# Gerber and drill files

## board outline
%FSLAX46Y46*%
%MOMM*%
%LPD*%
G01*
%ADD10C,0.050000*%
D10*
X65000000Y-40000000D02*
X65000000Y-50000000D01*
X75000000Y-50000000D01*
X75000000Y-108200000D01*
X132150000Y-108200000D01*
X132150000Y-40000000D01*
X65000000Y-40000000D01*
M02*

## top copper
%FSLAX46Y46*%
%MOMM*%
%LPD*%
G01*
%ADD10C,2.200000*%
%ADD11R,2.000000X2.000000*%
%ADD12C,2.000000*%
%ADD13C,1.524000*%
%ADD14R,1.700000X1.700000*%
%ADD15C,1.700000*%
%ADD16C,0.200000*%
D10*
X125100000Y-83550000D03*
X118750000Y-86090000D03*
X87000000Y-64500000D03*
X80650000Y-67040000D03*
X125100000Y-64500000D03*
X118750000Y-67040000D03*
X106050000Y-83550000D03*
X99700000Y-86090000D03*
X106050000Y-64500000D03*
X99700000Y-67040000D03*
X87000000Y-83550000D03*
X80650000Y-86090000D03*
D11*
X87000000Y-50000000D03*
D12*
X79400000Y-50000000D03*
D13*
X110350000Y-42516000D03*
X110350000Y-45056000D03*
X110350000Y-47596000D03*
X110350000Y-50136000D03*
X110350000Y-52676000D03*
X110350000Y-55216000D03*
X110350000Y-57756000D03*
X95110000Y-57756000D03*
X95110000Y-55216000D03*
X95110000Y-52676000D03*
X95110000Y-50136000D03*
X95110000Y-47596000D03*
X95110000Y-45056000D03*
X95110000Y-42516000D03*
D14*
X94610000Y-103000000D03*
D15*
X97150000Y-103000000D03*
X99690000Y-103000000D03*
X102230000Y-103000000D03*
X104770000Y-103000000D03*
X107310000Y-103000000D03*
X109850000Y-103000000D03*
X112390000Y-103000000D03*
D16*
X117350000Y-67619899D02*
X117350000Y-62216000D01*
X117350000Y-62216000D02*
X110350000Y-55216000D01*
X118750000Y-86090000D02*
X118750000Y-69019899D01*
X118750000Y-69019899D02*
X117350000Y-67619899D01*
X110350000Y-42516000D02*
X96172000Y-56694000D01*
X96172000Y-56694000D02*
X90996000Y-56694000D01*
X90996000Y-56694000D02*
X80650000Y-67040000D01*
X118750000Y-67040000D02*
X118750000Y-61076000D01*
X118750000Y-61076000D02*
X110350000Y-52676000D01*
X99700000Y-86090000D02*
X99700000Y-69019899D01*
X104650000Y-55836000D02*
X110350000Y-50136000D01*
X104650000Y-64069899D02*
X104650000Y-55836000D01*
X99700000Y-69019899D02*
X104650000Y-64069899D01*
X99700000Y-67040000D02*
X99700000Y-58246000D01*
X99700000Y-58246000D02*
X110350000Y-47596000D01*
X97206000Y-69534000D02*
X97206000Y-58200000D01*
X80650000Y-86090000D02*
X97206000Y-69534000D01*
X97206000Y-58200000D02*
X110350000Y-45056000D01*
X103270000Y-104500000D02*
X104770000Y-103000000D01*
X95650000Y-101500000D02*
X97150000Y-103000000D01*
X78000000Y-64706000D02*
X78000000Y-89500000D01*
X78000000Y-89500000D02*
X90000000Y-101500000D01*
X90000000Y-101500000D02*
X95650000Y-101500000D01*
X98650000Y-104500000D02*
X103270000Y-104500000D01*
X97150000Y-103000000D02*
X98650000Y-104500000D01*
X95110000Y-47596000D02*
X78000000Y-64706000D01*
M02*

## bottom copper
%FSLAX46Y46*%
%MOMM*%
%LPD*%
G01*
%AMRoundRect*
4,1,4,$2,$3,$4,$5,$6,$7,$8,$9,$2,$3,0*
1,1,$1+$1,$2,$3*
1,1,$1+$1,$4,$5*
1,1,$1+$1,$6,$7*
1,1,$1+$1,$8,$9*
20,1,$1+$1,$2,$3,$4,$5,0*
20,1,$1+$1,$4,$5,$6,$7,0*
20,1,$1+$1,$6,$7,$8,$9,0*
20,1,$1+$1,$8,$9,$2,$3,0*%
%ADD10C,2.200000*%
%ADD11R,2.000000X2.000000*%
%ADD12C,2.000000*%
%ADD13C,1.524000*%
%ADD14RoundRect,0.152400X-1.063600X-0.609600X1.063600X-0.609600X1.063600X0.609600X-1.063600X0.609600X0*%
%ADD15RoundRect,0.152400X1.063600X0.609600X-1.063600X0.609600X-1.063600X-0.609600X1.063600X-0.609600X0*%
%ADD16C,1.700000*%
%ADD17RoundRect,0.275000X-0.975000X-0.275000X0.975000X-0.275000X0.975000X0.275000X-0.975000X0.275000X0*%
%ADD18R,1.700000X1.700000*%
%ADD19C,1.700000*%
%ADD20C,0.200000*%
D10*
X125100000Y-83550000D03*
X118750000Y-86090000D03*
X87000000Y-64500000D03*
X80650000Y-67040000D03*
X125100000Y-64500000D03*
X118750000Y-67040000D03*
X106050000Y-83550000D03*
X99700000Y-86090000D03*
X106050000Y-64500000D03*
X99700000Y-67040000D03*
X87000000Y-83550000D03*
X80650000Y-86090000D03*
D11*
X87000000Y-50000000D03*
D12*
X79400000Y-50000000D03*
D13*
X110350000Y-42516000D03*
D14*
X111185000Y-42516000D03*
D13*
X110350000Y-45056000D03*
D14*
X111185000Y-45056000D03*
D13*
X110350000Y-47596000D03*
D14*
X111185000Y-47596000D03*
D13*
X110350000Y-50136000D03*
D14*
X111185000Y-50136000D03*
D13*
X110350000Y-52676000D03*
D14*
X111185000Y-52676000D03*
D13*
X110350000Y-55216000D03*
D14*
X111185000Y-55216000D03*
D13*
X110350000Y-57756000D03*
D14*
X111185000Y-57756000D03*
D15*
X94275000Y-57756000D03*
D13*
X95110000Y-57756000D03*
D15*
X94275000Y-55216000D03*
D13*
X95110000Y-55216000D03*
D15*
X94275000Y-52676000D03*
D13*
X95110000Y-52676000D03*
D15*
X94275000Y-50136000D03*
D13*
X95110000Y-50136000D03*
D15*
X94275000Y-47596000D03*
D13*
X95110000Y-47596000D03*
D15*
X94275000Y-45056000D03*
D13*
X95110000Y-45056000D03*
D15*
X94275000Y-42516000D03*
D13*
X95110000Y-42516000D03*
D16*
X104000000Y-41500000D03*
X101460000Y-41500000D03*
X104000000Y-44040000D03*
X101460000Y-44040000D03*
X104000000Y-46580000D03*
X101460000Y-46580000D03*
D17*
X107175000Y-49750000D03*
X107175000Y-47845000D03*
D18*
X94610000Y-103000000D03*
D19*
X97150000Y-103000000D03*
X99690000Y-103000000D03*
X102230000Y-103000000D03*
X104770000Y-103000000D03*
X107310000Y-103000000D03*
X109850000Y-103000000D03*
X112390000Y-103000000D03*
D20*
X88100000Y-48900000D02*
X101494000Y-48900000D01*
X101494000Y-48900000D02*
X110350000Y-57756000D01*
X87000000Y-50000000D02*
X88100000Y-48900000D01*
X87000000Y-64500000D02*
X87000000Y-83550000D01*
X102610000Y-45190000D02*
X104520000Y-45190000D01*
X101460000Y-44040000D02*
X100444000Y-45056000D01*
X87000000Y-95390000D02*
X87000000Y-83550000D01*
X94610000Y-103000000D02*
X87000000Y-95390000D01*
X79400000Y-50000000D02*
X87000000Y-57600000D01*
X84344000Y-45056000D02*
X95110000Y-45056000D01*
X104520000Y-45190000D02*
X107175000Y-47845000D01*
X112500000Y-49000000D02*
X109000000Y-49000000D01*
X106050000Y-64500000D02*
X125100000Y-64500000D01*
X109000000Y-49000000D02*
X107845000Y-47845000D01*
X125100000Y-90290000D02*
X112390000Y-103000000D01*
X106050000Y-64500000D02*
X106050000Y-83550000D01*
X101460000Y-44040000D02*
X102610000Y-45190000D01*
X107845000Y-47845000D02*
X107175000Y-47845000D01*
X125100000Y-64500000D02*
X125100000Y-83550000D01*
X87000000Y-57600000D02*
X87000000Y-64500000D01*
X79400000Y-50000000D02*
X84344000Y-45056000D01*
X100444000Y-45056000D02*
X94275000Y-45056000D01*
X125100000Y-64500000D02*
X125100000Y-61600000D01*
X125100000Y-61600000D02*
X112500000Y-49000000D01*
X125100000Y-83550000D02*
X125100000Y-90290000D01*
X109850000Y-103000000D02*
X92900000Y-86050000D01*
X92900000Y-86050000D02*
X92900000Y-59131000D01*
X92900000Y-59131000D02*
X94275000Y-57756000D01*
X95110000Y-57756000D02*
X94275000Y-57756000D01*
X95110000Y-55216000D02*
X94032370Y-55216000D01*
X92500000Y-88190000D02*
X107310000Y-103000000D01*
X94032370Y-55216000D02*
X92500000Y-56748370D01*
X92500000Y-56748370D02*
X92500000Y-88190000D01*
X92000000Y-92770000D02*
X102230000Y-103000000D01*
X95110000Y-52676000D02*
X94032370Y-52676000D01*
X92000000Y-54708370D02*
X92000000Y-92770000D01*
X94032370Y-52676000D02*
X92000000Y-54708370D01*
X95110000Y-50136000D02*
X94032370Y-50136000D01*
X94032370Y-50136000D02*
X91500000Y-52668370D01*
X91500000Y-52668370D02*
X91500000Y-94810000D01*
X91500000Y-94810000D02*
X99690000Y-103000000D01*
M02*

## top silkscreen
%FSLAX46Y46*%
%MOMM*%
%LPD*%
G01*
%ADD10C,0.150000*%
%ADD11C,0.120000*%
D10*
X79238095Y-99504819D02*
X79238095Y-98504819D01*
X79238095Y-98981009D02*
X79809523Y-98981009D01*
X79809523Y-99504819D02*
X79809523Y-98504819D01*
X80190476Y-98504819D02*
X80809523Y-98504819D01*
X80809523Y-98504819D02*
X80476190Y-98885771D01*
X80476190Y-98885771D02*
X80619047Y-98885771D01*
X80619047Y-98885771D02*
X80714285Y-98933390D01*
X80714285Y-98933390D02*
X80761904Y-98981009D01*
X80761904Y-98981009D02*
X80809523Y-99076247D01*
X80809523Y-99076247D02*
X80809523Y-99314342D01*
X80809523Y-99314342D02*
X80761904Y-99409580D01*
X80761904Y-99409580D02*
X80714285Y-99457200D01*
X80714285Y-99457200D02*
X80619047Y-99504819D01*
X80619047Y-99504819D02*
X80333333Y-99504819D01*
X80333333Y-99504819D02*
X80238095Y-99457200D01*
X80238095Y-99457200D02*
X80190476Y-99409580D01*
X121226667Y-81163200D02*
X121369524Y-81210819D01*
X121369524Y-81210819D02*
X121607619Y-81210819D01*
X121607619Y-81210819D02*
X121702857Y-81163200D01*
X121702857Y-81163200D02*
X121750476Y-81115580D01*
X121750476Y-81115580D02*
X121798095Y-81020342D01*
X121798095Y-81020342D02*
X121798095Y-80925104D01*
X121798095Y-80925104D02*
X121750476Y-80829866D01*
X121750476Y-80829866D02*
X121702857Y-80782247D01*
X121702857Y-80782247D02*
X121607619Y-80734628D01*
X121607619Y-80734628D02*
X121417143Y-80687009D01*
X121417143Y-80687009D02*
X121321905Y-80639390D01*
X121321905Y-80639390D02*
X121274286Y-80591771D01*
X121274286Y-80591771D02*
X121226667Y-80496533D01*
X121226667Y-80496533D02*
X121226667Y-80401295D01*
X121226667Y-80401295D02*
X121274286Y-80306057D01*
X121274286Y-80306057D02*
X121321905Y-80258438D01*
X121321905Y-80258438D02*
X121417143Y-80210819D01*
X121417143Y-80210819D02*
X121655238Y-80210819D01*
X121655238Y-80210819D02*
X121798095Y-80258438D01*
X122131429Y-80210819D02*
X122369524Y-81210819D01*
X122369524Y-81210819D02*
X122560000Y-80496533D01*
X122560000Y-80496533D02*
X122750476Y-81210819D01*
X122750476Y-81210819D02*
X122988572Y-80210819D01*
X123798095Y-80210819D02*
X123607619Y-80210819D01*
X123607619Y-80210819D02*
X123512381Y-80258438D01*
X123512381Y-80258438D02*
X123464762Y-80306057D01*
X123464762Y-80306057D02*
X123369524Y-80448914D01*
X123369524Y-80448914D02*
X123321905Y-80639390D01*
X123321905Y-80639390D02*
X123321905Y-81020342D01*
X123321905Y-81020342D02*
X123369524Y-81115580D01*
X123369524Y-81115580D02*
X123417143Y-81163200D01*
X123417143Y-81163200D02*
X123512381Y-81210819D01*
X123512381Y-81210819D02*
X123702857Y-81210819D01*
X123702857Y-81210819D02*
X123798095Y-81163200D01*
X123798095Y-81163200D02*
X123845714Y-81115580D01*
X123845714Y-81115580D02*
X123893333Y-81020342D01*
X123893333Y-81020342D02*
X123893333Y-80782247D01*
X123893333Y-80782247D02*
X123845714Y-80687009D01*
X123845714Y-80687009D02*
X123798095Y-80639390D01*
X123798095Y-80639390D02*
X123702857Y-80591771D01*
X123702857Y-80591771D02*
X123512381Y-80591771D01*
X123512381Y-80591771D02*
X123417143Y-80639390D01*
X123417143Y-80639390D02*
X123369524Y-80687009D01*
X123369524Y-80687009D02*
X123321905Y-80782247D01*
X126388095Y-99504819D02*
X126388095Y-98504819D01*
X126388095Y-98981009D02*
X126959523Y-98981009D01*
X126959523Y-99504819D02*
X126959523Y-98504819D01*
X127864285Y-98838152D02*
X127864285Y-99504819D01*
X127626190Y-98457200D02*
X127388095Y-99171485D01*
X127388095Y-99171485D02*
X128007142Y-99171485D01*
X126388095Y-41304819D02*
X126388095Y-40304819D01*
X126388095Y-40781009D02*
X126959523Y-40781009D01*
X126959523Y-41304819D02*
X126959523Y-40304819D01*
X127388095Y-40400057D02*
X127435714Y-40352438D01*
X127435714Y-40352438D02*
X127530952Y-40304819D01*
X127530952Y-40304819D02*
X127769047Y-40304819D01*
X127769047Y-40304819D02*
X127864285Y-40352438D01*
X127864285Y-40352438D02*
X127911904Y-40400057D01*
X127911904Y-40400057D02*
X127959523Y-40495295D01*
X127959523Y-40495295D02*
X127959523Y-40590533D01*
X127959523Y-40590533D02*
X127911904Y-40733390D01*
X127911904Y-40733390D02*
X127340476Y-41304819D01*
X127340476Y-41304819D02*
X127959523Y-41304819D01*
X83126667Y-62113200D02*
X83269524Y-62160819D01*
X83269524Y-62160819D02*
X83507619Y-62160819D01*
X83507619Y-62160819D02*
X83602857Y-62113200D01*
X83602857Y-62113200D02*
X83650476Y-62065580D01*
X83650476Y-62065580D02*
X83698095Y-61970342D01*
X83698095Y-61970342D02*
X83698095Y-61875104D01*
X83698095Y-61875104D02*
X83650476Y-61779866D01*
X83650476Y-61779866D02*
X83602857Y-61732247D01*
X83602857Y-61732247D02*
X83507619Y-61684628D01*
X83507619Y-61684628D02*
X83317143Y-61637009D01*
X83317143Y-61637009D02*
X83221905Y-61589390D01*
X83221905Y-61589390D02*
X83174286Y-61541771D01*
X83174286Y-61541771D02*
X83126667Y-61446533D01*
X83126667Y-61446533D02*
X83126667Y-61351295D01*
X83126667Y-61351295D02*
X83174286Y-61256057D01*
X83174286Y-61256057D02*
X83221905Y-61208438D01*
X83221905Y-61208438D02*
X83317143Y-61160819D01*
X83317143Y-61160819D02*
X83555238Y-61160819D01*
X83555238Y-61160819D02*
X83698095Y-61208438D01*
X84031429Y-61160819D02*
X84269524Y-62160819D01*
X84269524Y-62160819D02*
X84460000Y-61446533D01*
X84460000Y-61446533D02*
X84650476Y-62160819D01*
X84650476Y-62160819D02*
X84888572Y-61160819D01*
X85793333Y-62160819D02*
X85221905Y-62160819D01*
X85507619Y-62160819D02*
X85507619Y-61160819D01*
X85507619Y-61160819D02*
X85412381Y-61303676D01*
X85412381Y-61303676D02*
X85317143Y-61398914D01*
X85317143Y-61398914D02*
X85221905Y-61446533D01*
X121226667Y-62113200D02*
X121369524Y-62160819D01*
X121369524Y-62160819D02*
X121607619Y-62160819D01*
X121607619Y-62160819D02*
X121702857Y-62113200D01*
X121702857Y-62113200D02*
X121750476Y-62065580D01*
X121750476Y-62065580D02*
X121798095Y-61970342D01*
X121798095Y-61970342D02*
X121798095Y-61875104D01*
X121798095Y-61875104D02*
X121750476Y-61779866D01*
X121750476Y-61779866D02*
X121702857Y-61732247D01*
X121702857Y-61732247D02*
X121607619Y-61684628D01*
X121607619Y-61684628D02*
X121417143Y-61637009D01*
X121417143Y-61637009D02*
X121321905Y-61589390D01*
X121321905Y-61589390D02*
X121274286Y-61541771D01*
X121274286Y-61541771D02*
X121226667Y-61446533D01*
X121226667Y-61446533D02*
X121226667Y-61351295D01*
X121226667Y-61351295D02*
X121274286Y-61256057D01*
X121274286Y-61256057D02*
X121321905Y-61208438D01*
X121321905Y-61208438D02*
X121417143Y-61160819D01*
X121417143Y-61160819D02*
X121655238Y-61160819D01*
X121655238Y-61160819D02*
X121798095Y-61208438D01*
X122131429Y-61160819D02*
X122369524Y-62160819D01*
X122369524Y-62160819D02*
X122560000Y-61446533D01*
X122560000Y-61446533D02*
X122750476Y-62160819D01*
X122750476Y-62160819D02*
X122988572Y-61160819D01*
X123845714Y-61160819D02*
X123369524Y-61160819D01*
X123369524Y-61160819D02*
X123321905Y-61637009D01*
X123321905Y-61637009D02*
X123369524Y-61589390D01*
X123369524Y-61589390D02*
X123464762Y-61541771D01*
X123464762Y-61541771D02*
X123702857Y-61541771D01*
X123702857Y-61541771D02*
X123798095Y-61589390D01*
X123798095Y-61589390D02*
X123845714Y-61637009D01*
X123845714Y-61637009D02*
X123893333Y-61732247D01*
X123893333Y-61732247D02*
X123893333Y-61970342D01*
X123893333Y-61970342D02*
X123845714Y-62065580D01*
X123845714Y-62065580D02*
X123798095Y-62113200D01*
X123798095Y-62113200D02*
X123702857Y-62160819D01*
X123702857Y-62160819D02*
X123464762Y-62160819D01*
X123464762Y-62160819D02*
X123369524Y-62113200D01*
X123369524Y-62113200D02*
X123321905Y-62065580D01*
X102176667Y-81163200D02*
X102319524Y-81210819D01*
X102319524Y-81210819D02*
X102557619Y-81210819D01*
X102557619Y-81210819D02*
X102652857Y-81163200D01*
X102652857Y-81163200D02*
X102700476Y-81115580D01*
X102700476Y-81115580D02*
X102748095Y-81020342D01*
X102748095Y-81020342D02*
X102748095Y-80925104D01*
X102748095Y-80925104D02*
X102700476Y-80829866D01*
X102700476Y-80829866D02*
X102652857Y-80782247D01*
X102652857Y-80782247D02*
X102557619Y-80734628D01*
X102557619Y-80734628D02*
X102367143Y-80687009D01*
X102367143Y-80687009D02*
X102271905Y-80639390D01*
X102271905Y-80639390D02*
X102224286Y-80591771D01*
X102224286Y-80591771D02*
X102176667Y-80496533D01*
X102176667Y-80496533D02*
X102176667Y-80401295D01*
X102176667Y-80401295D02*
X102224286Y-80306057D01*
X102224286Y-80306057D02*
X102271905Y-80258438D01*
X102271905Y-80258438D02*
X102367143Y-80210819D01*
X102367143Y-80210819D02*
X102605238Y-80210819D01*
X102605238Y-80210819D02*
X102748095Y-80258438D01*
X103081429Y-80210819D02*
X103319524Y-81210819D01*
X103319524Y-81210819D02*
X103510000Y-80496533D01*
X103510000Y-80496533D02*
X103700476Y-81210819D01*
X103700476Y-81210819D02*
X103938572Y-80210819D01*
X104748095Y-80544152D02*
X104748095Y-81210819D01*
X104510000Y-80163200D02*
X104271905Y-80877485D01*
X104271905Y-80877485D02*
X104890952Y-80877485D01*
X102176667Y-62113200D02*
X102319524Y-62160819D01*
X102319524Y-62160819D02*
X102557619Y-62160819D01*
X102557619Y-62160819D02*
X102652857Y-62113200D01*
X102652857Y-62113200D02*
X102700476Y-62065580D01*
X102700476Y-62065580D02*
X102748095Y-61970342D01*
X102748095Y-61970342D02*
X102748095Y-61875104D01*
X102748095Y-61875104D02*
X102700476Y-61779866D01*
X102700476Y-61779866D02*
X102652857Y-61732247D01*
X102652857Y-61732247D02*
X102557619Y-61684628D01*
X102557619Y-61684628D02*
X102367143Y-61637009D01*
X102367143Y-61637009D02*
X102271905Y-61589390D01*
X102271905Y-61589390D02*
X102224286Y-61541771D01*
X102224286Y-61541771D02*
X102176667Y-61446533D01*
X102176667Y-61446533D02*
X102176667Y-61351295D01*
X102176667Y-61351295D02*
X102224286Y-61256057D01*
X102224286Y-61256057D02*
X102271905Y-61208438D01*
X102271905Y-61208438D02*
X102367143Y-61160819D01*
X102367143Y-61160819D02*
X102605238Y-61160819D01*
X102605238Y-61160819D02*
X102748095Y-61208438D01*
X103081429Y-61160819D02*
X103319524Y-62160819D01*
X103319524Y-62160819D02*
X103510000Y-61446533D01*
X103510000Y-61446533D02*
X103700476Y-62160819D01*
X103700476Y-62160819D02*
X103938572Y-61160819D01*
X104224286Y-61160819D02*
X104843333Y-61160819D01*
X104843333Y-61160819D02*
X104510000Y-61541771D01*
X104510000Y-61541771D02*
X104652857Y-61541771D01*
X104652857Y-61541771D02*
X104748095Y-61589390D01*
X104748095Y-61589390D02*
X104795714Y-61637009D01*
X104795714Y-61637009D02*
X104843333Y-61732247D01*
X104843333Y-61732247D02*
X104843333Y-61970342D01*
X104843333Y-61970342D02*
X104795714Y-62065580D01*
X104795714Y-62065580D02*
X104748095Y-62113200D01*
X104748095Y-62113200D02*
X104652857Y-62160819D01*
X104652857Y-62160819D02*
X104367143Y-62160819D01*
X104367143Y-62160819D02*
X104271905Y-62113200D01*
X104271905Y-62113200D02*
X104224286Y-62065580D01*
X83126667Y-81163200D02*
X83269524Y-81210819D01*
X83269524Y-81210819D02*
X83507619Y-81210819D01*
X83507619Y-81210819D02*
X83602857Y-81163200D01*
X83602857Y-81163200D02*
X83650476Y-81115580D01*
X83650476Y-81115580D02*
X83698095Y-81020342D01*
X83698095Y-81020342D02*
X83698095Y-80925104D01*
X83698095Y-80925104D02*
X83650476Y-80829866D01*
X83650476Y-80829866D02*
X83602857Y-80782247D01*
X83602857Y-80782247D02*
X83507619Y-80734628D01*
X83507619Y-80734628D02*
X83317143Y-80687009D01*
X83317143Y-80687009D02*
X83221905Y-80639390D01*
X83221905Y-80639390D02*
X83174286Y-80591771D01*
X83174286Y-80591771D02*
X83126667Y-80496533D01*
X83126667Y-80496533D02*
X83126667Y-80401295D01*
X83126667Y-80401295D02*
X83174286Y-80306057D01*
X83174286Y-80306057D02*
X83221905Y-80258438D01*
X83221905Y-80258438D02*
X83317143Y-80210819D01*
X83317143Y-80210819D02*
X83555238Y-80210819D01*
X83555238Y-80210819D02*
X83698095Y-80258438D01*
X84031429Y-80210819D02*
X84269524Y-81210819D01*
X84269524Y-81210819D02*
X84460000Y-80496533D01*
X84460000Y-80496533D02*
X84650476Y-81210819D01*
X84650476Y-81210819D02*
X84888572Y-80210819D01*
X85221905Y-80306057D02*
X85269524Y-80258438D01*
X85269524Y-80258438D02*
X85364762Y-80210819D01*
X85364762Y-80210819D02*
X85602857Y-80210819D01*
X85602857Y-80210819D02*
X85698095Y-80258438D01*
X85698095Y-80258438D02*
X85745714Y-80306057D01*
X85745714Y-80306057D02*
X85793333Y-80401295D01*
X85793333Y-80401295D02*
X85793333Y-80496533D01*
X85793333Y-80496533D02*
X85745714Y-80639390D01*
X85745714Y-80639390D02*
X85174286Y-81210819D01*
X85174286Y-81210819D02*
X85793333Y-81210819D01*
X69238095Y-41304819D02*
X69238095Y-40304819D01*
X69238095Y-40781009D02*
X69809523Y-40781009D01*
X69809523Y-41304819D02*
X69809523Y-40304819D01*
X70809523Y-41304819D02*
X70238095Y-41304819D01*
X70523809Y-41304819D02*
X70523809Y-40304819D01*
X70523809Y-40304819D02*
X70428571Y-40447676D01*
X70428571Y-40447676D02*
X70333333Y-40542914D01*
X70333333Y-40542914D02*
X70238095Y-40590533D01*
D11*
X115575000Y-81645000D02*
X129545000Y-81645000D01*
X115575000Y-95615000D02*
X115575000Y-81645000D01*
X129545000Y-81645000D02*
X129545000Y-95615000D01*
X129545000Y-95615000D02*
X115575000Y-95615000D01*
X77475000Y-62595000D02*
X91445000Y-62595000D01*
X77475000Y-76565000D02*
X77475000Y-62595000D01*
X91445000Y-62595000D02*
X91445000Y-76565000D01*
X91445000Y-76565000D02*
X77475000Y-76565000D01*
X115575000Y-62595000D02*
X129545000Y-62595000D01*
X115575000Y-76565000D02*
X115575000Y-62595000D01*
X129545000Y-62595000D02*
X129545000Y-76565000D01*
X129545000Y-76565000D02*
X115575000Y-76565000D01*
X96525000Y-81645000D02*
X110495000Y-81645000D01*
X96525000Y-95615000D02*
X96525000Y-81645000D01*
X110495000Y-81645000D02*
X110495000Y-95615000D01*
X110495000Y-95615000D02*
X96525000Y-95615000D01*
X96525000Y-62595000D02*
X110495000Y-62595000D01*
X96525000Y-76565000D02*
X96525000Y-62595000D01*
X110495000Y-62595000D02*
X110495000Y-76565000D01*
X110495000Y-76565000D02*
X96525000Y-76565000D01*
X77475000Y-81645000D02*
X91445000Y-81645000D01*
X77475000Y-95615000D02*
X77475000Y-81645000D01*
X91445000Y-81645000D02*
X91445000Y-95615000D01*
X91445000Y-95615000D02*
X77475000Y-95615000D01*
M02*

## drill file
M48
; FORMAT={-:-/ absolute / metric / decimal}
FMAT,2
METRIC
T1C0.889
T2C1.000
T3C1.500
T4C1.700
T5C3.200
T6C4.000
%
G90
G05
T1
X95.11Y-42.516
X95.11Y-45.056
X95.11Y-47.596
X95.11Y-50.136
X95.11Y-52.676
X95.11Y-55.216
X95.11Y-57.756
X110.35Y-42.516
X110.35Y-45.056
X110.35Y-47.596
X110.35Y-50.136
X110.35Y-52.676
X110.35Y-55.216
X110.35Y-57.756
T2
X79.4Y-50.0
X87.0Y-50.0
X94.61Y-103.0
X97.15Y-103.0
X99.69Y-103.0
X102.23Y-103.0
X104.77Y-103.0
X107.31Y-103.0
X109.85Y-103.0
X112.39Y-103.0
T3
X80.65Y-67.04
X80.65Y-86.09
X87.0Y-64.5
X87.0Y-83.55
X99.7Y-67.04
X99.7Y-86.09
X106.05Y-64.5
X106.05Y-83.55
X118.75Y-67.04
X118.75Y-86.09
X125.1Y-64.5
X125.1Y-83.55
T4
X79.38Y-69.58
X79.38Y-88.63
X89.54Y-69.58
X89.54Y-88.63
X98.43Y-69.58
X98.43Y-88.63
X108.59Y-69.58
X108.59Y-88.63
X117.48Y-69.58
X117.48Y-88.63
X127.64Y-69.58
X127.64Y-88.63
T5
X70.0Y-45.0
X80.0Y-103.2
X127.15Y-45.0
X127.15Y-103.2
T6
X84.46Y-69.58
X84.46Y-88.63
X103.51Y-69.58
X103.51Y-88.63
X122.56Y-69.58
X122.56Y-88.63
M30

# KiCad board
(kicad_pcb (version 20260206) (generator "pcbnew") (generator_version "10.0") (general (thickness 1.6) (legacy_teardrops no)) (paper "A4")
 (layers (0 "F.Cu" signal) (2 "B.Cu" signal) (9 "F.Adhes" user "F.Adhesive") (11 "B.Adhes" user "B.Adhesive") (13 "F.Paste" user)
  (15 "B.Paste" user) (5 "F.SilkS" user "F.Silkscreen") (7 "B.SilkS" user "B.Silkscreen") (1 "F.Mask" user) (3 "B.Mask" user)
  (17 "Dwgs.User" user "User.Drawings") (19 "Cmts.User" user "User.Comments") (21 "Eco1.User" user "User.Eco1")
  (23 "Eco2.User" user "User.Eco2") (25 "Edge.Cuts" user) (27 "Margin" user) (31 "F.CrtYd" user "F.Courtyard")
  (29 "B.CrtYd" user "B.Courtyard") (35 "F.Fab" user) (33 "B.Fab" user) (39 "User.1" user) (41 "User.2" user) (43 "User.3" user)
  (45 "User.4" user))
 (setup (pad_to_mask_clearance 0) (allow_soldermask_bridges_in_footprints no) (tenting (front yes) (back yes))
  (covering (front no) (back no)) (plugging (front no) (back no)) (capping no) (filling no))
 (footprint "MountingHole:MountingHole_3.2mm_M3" (layer "F.Cu") (at 80 103.2)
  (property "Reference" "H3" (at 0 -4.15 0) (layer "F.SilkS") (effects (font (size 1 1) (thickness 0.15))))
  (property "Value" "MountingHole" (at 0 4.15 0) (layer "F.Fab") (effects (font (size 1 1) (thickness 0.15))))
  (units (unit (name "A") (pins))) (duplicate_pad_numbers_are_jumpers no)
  (pad "" np_thru_hole circle (at 0 0) (size 3.2 3.2) (drill 3.2) (layers "*.Cu" "*.Mask")))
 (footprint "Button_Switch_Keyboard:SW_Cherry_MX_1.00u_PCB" (layer "F.Cu") (at 125.1 83.55)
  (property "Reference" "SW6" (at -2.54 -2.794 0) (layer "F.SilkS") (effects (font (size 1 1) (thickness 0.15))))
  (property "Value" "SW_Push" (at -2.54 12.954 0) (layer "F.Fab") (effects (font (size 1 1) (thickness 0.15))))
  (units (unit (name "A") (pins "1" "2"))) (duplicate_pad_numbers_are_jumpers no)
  (fp_line (start -9.525 -1.905) (end 4.445 -1.905) (stroke (width 0.12) (type solid)) (layer "F.SilkS"))
  (fp_line (start -9.525 12.065) (end -9.525 -1.905) (stroke (width 0.12) (type solid)) (layer "F.SilkS"))
  (fp_line (start 4.445 -1.905) (end 4.445 12.065) (stroke (width 0.12) (type solid)) (layer "F.SilkS"))
  (fp_line (start 4.445 12.065) (end -9.525 12.065) (stroke (width 0.12) (type solid)) (layer "F.SilkS"))
  (pad "" np_thru_hole circle (at -7.62 5.08) (size 1.7 1.7) (drill 1.7) (layers "*.Cu" "*.Mask"))
  (pad "" np_thru_hole circle (at -2.54 5.08) (size 4 4) (drill 4) (layers "*.Cu" "*.Mask"))
  (pad "" np_thru_hole circle (at 2.54 5.08) (size 1.7 1.7) (drill 1.7) (layers "*.Cu" "*.Mask"))
  (pad "1" thru_hole circle (at 0 0) (size 2.2 2.2) (drill 1.5) (layers "*.Cu" "*.Mask") (remove_unused_layers no) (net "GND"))
  (pad "2" thru_hole circle (at -6.35 2.54) (size 2.2 2.2) (drill 1.5) (layers "*.Cu" "*.Mask") (remove_unused_layers no)
   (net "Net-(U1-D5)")))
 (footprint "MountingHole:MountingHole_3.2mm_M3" (layer "F.Cu") (at 127.15 103.2)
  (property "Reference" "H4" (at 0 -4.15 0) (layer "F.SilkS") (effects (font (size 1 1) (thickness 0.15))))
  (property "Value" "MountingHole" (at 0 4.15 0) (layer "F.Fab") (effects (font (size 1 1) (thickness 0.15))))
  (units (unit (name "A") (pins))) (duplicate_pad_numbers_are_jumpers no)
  (pad "" np_thru_hole circle (at 0 0) (size 3.2 3.2) (drill 3.2) (layers "*.Cu" "*.Mask")))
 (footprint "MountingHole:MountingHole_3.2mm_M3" (layer "F.Cu") (at 127.15 45)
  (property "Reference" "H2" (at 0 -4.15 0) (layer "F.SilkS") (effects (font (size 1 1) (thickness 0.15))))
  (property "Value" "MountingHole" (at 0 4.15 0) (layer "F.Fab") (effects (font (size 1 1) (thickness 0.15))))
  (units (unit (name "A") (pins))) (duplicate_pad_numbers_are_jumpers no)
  (pad "" np_thru_hole circle (at 0 0) (size 3.2 3.2) (drill 3.2) (layers "*.Cu" "*.Mask")))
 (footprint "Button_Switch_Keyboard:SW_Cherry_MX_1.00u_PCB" (layer "F.Cu") (at 87 64.5)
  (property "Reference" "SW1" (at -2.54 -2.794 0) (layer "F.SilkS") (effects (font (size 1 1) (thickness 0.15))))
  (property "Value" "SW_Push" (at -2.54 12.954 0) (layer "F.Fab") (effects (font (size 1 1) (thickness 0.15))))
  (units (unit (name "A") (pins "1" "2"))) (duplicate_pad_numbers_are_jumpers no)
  (fp_line (start -9.525 -1.905) (end 4.445 -1.905) (stroke (width 0.12) (type solid)) (layer "F.SilkS"))
  (fp_line (start -9.525 12.065) (end -9.525 -1.905) (stroke (width 0.12) (type solid)) (layer "F.SilkS"))
  (fp_line (start 4.445 -1.905) (end 4.445 12.065) (stroke (width 0.12) (type solid)) (layer "F.SilkS"))
  (fp_line (start 4.445 12.065) (end -9.525 12.065) (stroke (width 0.12) (type solid)) (layer "F.SilkS"))
  (pad "" np_thru_hole circle (at -7.62 5.08) (size 1.7 1.7) (drill 1.7) (layers "*.Cu" "*.Mask"))
  (pad "" np_thru_hole circle (at -2.54 5.08) (size 4 4) (drill 4) (layers "*.Cu" "*.Mask"))
  (pad "" np_thru_hole circle (at 2.54 5.08) (size 1.7 1.7) (drill 1.7) (layers "*.Cu" "*.Mask"))
  (pad "1" thru_hole circle (at 0 0) (size 2.2 2.2) (drill 1.5) (layers "*.Cu" "*.Mask") (remove_unused_layers no) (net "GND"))
  (pad "2" thru_hole circle (at -6.35 2.54) (size 2.2 2.2) (drill 1.5) (layers "*.Cu" "*.Mask") (remove_unused_layers no)
   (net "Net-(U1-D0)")))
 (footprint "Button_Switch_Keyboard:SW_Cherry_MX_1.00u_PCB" (layer "F.Cu") (at 125.1 64.5)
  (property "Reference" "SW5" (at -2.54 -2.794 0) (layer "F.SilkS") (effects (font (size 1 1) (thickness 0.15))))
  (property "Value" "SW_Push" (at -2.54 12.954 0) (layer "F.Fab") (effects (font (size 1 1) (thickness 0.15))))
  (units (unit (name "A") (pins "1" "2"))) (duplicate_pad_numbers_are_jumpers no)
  (fp_line (start -9.525 -1.905) (end 4.445 -1.905) (stroke (width 0.12) (type solid)) (layer "F.SilkS"))
  (fp_line (start -9.525 12.065) (end -9.525 -1.905) (stroke (width 0.12) (type solid)) (layer "F.SilkS"))
  (fp_line (start 4.445 -1.905) (end 4.445 12.065) (stroke (width 0.12) (type solid)) (layer "F.SilkS"))
  (fp_line (start 4.445 12.065) (end -9.525 12.065) (stroke (width 0.12) (type solid)) (layer "F.SilkS"))
  (pad "" np_thru_hole circle (at -7.62 5.08) (size 1.7 1.7) (drill 1.7) (layers "*.Cu" "*.Mask"))
  (pad "" np_thru_hole circle (at -2.54 5.08) (size 4 4) (drill 4) (layers "*.Cu" "*.Mask"))
  (pad "" np_thru_hole circle (at 2.54 5.08) (size 1.7 1.7) (drill 1.7) (layers "*.Cu" "*.Mask"))
  (pad "1" thru_hole circle (at 0 0) (size 2.2 2.2) (drill 1.5) (layers "*.Cu" "*.Mask") (remove_unused_layers no) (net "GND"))
  (pad "2" thru_hole circle (at -6.35 2.54) (size 2.2 2.2) (drill 1.5) (layers "*.Cu" "*.Mask") (remove_unused_layers no)
   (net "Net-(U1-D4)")))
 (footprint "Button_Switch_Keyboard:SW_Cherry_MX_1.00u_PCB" (layer "F.Cu") (at 106.05 83.55)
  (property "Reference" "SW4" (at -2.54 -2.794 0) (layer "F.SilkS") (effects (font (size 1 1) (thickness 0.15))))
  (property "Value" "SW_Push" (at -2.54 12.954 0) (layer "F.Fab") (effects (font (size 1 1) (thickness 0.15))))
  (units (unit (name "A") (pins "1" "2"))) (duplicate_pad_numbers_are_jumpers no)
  (fp_line (start -9.525 -1.905) (end 4.445 -1.905) (stroke (width 0.12) (type solid)) (layer "F.SilkS"))
  (fp_line (start -9.525 12.065) (end -9.525 -1.905) (stroke (width 0.12) (type solid)) (layer "F.SilkS"))
  (fp_line (start 4.445 -1.905) (end 4.445 12.065) (stroke (width 0.12) (type solid)) (layer "F.SilkS"))
  (fp_line (start 4.445 12.065) (end -9.525 12.065) (stroke (width 0.12) (type solid)) (layer "F.SilkS"))
  (pad "" np_thru_hole circle (at -7.62 5.08) (size 1.7 1.7) (drill 1.7) (layers "*.Cu" "*.Mask"))
  (pad "" np_thru_hole circle (at -2.54 5.08) (size 4 4) (drill 4) (layers "*.Cu" "*.Mask"))
  (pad "" np_thru_hole circle (at 2.54 5.08) (size 1.7 1.7) (drill 1.7) (layers "*.Cu" "*.Mask"))
  (pad "1" thru_hole circle (at 0 0) (size 2.2 2.2) (drill 1.5) (layers "*.Cu" "*.Mask") (remove_unused_layers no) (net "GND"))
  (pad "2" thru_hole circle (at -6.35 2.54) (size 2.2 2.2) (drill 1.5) (layers "*.Cu" "*.Mask") (remove_unused_layers no)
   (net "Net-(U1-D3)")))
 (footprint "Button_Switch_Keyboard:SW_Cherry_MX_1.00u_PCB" (layer "F.Cu") (at 106.05 64.5)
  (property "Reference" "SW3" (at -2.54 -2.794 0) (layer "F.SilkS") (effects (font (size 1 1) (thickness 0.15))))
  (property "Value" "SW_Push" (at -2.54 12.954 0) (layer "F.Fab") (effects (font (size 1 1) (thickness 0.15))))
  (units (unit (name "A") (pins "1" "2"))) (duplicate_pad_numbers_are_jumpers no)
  (fp_line (start -9.525 -1.905) (end 4.445 -1.905) (stroke (width 0.12) (type solid)) (layer "F.SilkS"))
  (fp_line (start -9.525 12.065) (end -9.525 -1.905) (stroke (width 0.12) (type solid)) (layer "F.SilkS"))
  (fp_line (start 4.445 -1.905) (end 4.445 12.065) (stroke (width 0.12) (type solid)) (layer "F.SilkS"))
  (fp_line (start 4.445 12.065) (end -9.525 12.065) (stroke (width 0.12) (type solid)) (layer "F.SilkS"))
  (pad "" np_thru_hole circle (at -7.62 5.08) (size 1.7 1.7) (drill 1.7) (layers "*.Cu" "*.Mask"))
  (pad "" np_thru_hole circle (at -2.54 5.08) (size 4 4) (drill 4) (layers "*.Cu" "*.Mask"))
  (pad "" np_thru_hole circle (at 2.54 5.08) (size 1.7 1.7) (drill 1.7) (layers "*.Cu" "*.Mask"))
  (pad "1" thru_hole circle (at 0 0) (size 2.2 2.2) (drill 1.5) (layers "*.Cu" "*.Mask") (remove_unused_layers no) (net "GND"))
  (pad "2" thru_hole circle (at -6.35 2.54) (size 2.2 2.2) (drill 1.5) (layers "*.Cu" "*.Mask") (remove_unused_layers no)
   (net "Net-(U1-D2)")))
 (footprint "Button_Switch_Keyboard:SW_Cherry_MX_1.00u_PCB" (layer "F.Cu") (at 87 83.55)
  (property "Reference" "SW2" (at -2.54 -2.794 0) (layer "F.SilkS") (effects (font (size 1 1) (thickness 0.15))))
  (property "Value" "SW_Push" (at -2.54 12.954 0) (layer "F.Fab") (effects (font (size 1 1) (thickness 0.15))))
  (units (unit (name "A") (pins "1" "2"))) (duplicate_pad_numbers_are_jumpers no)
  (fp_line (start -9.525 -1.905) (end 4.445 -1.905) (stroke (width 0.12) (type solid)) (layer "F.SilkS"))
  (fp_line (start -9.525 12.065) (end -9.525 -1.905) (stroke (width 0.12) (type solid)) (layer "F.SilkS"))
  (fp_line (start 4.445 -1.905) (end 4.445 12.065) (stroke (width 0.12) (type solid)) (layer "F.SilkS"))
  (fp_line (start 4.445 12.065) (end -9.525 12.065) (stroke (width 0.12) (type solid)) (layer "F.SilkS"))
  (pad "" np_thru_hole circle (at -7.62 5.08) (size 1.7 1.7) (drill 1.7) (layers "*.Cu" "*.Mask"))
  (pad "" np_thru_hole circle (at -2.54 5.08) (size 4 4) (drill 4) (layers "*.Cu" "*.Mask"))
  (pad "" np_thru_hole circle (at 2.54 5.08) (size 1.7 1.7) (drill 1.7) (layers "*.Cu" "*.Mask"))
  (pad "1" thru_hole circle (at 0 0) (size 2.2 2.2) (drill 1.5) (layers "*.Cu" "*.Mask") (remove_unused_layers no) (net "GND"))
  (pad "2" thru_hole circle (at -6.35 2.54) (size 2.2 2.2) (drill 1.5) (layers "*.Cu" "*.Mask") (remove_unused_layers no)
   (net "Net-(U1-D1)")))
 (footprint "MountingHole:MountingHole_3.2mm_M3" (layer "F.Cu") (at 70 45)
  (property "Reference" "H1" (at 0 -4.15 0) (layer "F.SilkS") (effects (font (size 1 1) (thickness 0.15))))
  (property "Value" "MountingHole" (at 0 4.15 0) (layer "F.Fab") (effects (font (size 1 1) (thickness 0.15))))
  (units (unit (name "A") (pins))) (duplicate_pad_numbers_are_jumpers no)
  (pad "" np_thru_hole circle (at 0 0) (size 3.2 3.2) (drill 3.2) (layers "*.Cu" "*.Mask")))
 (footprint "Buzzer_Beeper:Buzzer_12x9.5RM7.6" (layer "B.Cu") (at 87 50 180)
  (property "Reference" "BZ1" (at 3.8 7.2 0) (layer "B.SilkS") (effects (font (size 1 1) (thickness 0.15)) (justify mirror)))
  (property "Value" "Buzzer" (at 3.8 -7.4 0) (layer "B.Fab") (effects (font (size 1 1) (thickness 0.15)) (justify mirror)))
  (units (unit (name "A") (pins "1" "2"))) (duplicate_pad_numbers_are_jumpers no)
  (pad "1" thru_hole rect (at 0 0 180) (size 2 2) (drill 1) (layers "*.Cu" "*.Mask") (remove_unused_layers no) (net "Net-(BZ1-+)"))
  (pad "2" thru_hole circle (at 7.6 0 180) (size 2 2) (drill 1) (layers "*.Cu" "*.Mask") (remove_unused_layers no) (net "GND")))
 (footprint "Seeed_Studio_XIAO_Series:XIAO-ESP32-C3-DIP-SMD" (layer "B.Cu") (at 102.73 50.136 90)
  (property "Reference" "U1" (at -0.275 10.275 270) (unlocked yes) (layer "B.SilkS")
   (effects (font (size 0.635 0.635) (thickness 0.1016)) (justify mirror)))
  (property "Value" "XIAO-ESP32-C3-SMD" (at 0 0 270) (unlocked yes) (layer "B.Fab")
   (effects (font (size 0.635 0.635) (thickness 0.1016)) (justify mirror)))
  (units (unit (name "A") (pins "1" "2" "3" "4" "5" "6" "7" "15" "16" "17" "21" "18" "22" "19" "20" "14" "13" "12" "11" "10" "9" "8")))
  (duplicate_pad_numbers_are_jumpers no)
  (pad "1" thru_hole circle (at 7.62 7.62) (size 1.524 1.524) (drill 0.889) (layers "*.Cu" "*.Mask") (remove_unused_layers no)
   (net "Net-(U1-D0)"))
  (pad "1" smd roundrect (at 7.62 8.455) (size 2.432 1.524) (layers "B.Cu" "B.Mask") (roundrect_rratio 0.1) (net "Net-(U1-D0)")
   (thermal_bridge_angle 45))
  (pad "2" thru_hole circle (at 5.08 7.62) (size 1.524 1.524) (drill 0.889) (layers "*.Cu" "*.Mask") (remove_unused_layers no)
   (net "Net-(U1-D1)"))
  (pad "2" smd roundrect (at 5.08 8.455) (size 2.432 1.524) (layers "B.Cu" "B.Mask") (roundrect_rratio 0.1) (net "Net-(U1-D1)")
   (thermal_bridge_angle 45))
  (pad "3" thru_hole circle (at 2.54 7.62) (size 1.524 1.524) (drill 0.889) (layers "*.Cu" "*.Mask") (remove_unused_layers no)
   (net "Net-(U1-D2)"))
  (pad "3" smd roundrect (at 2.54 8.455) (size 2.432 1.524) (layers "B.Cu" "B.Mask") (roundrect_rratio 0.1) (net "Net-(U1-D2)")
   (thermal_bridge_angle 45))
  (pad "4" thru_hole circle (at 0 7.62) (size 1.524 1.524) (drill 0.889) (layers "*.Cu" "*.Mask") (remove_unused_layers no)
   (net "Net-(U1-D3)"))
  (pad "4" smd roundrect (at 0 8.455) (size 2.432 1.524) (layers "B.Cu" "B.Mask") (roundrect_rratio 0.1) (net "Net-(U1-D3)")
   (thermal_bridge_angle 45))
  (pad "5" thru_hole circle (at -2.54 7.62) (size 1.524 1.524) (drill 0.889) (layers "*.Cu" "*.Mask") (remove_unused_layers no)
   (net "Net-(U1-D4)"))
  (pad "5" smd roundrect (at -2.54 8.455) (size 2.432 1.524) (layers "B.Cu" "B.Mask") (roundrect_rratio 0.1) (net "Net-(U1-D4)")
   (thermal_bridge_angle 45))
  (pad "6" thru_hole circle (at -5.08 7.62) (size 1.524 1.524) (drill 0.889) (layers "*.Cu" "*.Mask") (remove_unused_layers no)
   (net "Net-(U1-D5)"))
  (pad "6" smd roundrect (at -5.08 8.455) (size 2.432 1.524) (layers "B.Cu" "B.Mask") (roundrect_rratio 0.1) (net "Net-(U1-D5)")
   (thermal_bridge_angle 45))
  (pad "7" thru_hole circle (at -7.62 7.62) (size 1.524 1.524) (drill 0.889) (layers "*.Cu" "*.Mask") (remove_unused_layers no)
   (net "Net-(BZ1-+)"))
  (pad "7" smd roundrect (at -7.62 8.455) (size 2.432 1.524) (layers "B.Cu" "B.Mask") (roundrect_rratio 0.1) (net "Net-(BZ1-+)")
   (thermal_bridge_angle 45))
  (pad "8" smd roundrect (at -7.62 -8.455 180) (size 2.432 1.524) (layers "B.Cu" "B.Mask") (roundrect_rratio 0.1) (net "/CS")
   (thermal_bridge_angle 45))
  (pad "8" thru_hole circle (at -7.62 -7.62 180) (size 1.524 1.524) (drill 0.889) (layers "*.Cu" "*.Mask") (remove_unused_layers no)
   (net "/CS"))
  (pad "9" smd roundrect (at -5.08 -8.455 180) (size 2.432 1.524) (layers "B.Cu" "B.Mask") (roundrect_rratio 0.1) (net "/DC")
   (thermal_bridge_angle 45))
  (pad "9" thru_hole circle (at -5.08 -7.62 180) (size 1.524 1.524) (drill 0.889) (layers "*.Cu" "*.Mask") (remove_unused_layers no)
   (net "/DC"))
  (pad "10" smd roundrect (at -2.54 -8.455 180) (size 2.432 1.524) (layers "B.Cu" "B.Mask") (roundrect_rratio 0.1) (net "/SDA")
   (thermal_bridge_angle 45))
  (pad "10" thru_hole circle (at -2.54 -7.62 180) (size 1.524 1.524) (drill 0.889) (layers "*.Cu" "*.Mask") (remove_unused_layers no)
   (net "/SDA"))
  (pad "11" smd roundrect (at 0 -8.455 180) (size 2.432 1.524) (layers "B.Cu" "B.Mask") (roundrect_rratio 0.1) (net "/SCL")
   (thermal_bridge_angle 45))
  (pad "11" thru_hole circle (at 0 -7.62 180) (size 1.524 1.524) (drill 0.889) (layers "*.Cu" "*.Mask") (remove_unused_layers no)
   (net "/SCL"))
  (pad "12" smd roundrect (at 2.54 -8.455 180) (size 2.432 1.524) (layers "B.Cu" "B.Mask") (roundrect_rratio 0.1) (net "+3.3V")
   (thermal_bridge_angle 45))
  (pad "12" thru_hole circle (at 2.54 -7.62 180) (size 1.524 1.524) (drill 0.889) (layers "*.Cu" "*.Mask") (remove_unused_layers no)
   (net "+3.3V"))
  (pad "13" smd roundrect (at 5.08 -8.455 180) (size 2.432 1.524) (layers "B.Cu" "B.Mask") (roundrect_rratio 0.1) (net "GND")
   (thermal_bridge_angle 45))
  (pad "13" thru_hole circle (at 5.08 -7.62 180) (size 1.524 1.524) (drill 0.889) (layers "*.Cu" "*.Mask") (remove_unused_layers no)
   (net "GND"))
  (pad "14" smd roundrect (at 7.62 -8.455 180) (size 2.432 1.524) (layers "B.Cu" "B.Mask") (roundrect_rratio 0.1)
   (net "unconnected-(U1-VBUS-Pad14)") (thermal_bridge_angle 45))
  (pad "14" thru_hole circle (at 7.62 -7.62 180) (size 1.524 1.524) (drill 0.889) (layers "*.Cu" "*.Mask") (remove_unused_layers no)
   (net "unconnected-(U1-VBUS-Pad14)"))
  (pad "15" smd circle (at 8.636 1.27 180) (size 1.7 1.7) (layers "B.Cu" "B.Mask" "B.Paste") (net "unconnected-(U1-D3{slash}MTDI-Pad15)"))
  (pad "16" smd circle (at 8.636 -1.27 180) (size 1.7 1.7) (layers "B.Cu" "B.Mask" "B.Paste") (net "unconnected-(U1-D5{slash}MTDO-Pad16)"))
  (pad "17" smd circle (at 6.096 1.27 180) (size 1.7 1.7) (layers "B.Cu" "B.Mask" "B.Paste") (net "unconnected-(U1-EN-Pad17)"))
  (pad "18" smd circle (at 6.096 -1.27 180) (size 1.7 1.7) (layers "B.Cu" "B.Mask" "B.Paste") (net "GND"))
  (pad "19" smd circle (at 3.556 1.27 180) (size 1.7 1.7) (layers "B.Cu" "B.Mask" "B.Paste") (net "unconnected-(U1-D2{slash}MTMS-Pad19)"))
  (pad "20" smd circle (at 3.556 -1.27 180) (size 1.7 1.7) (layers "B.Cu" "B.Mask" "B.Paste") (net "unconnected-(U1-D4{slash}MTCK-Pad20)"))
  (pad "21" smd roundrect (at 0.386 4.445) (size 2.5 1.1) (layers "B.Cu" "B.Mask" "B.Paste") (roundrect_rratio 0.25)
   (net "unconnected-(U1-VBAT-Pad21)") (thermal_bridge_angle 45))
  (pad "22" smd roundrect (at 2.291 4.445) (size 2.5 1.1) (layers "B.Cu" "B.Mask" "B.Paste") (roundrect_rratio 0.25) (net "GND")
   (thermal_bridge_angle 45)))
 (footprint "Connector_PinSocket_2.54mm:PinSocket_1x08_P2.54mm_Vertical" (layer "B.Cu") (at 94.61 103 -90)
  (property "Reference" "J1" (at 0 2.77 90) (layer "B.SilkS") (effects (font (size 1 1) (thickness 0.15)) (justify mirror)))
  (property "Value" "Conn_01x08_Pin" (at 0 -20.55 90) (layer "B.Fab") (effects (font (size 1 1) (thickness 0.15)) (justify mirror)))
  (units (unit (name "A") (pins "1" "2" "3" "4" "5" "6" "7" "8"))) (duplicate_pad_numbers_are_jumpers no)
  (pad "1" thru_hole rect (at 0 0 270) (size 1.7 1.7) (drill 1) (layers "*.Cu" "*.Mask") (remove_unused_layers no) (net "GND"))
  (pad "2" thru_hole circle (at 0 -2.54 270) (size 1.7 1.7) (drill 1) (layers "*.Cu" "*.Mask") (remove_unused_layers no) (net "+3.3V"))
  (pad "3" thru_hole circle (at 0 -5.08 270) (size 1.7 1.7) (drill 1) (layers "*.Cu" "*.Mask") (remove_unused_layers no) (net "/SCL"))
  (pad "4" thru_hole circle (at 0 -7.62 270) (size 1.7 1.7) (drill 1) (layers "*.Cu" "*.Mask") (remove_unused_layers no) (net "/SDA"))
  (pad "5" thru_hole circle (at 0 -10.16 270) (size 1.7 1.7) (drill 1) (layers "*.Cu" "*.Mask") (remove_unused_layers no) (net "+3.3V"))
  (pad "6" thru_hole circle (at 0 -12.7 270) (size 1.7 1.7) (drill 1) (layers "*.Cu" "*.Mask") (remove_unused_layers no) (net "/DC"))
  (pad "7" thru_hole circle (at 0 -15.24 270) (size 1.7 1.7) (drill 1) (layers "*.Cu" "*.Mask") (remove_unused_layers no) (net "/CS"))
  (pad "8" thru_hole circle (at 0 -17.78 270) (size 1.7 1.7) (drill 1) (layers "*.Cu" "*.Mask") (remove_unused_layers no) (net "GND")))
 (gr_poly
  (pts (xy 65 40) (xy 65 50) (xy 75 50) (xy 75 108.2) (xy 132.15 108.2) (xy 132.15 40)) (stroke (width 0.05) (type solid)) (fill no)
  (layer "Edge.Cuts"))
 (segment (start 88.1 48.9) (end 101.494 48.9) (width 0.2) (layer "B.Cu") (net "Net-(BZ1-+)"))
 (segment (start 101.494 48.9) (end 110.35 57.756) (width 0.2) (layer "B.Cu") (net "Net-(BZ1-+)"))
 (segment (start 87 50) (end 88.1 48.9) (width 0.2) (layer "B.Cu") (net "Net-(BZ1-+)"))
 (segment (start 87 64.5) (end 87 83.55) (width 0.2) (layer "B.Cu") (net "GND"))
 (segment (start 102.61 45.19) (end 104.52 45.19) (width 0.2) (layer "B.Cu") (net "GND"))
 (segment (start 101.46 44.04) (end 100.444 45.056) (width 0.2) (layer "B.Cu") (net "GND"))
 (segment (start 87 95.39) (end 87 83.55) (width 0.2) (layer "B.Cu") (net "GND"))
 (segment (start 94.61 103) (end 87 95.39) (width 0.2) (layer "B.Cu") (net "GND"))
 (segment (start 79.4 50) (end 87 57.6) (width 0.2) (layer "B.Cu") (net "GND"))
 (segment (start 84.344 45.056) (end 95.11 45.056) (width 0.2) (layer "B.Cu") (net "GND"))
 (segment (start 104.52 45.19) (end 107.175 47.845) (width 0.2) (layer "B.Cu") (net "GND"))
 (segment (start 112.5 49) (end 109 49) (width 0.2) (layer "B.Cu") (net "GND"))
 (segment (start 106.05 64.5) (end 125.1 64.5) (width 0.2) (layer "B.Cu") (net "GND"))
 (segment (start 109 49) (end 107.845 47.845) (width 0.2) (layer "B.Cu") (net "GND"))
 (segment (start 125.1 90.29) (end 112.39 103) (width 0.2) (layer "B.Cu") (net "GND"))
 (segment (start 106.05 64.5) (end 106.05 83.55) (width 0.2) (layer "B.Cu") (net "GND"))
 (segment (start 101.46 44.04) (end 102.61 45.19) (width 0.2) (layer "B.Cu") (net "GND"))
 (segment (start 107.845 47.845) (end 107.175 47.845) (width 0.2) (layer "B.Cu") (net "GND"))
 (segment (start 125.1 64.5) (end 125.1 83.55) (width 0.2) (layer "B.Cu") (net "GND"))
 (segment (start 87 57.6) (end 87 64.5) (width 0.2) (layer "B.Cu") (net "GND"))
 (segment (start 79.4 50) (end 84.344 45.056) (width 0.2) (layer "B.Cu") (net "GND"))
 (segment (start 100.444 45.056) (end 94.275 45.056) (width 0.2) (layer "B.Cu") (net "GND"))
 (segment (start 125.1 64.5) (end 125.1 61.6) (width 0.2) (layer "B.Cu") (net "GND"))
 (segment (start 125.1 61.6) (end 112.5 49) (width 0.2) (layer "B.Cu") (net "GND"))
 (segment (start 125.1 83.55) (end 125.1 90.29) (width 0.2) (layer "B.Cu") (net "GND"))
 (segment (start 117.35 67.619899) (end 117.35 62.216) (width 0.2) (layer "F.Cu") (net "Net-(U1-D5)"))
 (segment (start 117.35 62.216) (end 110.35 55.216) (width 0.2) (layer "F.Cu") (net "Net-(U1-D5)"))
 (segment (start 118.75 86.09) (end 118.75 69.019899) (width 0.2) (layer "F.Cu") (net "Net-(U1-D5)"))
 (segment (start 118.75 69.019899) (end 117.35 67.619899) (width 0.2) (layer "F.Cu") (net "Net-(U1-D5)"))
 (segment (start 110.35 42.516) (end 96.172 56.694) (width 0.2) (layer "F.Cu") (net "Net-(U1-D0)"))
 (segment (start 96.172 56.694) (end 90.996 56.694) (width 0.2) (layer "F.Cu") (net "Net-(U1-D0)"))
 (segment (start 90.996 56.694) (end 80.65 67.04) (width 0.2) (layer "F.Cu") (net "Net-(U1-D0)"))
 (segment (start 118.75 67.04) (end 118.75 61.076) (width 0.2) (layer "F.Cu") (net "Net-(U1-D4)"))
 (segment (start 118.75 61.076) (end 110.35 52.676) (width 0.2) (layer "F.Cu") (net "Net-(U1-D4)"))
 (segment (start 99.7 86.09) (end 99.7 69.019899) (width 0.2) (layer "F.Cu") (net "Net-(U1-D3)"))
 (segment (start 104.65 55.836) (end 110.35 50.136) (width 0.2) (layer "F.Cu") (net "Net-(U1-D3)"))
 (segment (start 104.65 64.069899) (end 104.65 55.836) (width 0.2) (layer "F.Cu") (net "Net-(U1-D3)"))
 (segment (start 99.7 69.019899) (end 104.65 64.069899) (width 0.2) (layer "F.Cu") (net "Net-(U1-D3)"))
 (segment (start 99.7 67.04) (end 99.7 58.246) (width 0.2) (layer "F.Cu") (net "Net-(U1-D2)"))
 (segment (start 99.7 58.246) (end 110.35 47.596) (width 0.2) (layer "F.Cu") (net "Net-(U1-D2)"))
 (segment (start 97.206 69.534) (end 97.206 58.2) (width 0.2) (layer "F.Cu") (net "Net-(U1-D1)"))
 (segment (start 80.65 86.09) (end 97.206 69.534) (width 0.2) (layer "F.Cu") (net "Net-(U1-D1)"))
 (segment (start 97.206 58.2) (end 110.35 45.056) (width 0.2) (layer "F.Cu") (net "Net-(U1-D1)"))
 (segment (start 109.85 103) (end 92.9 86.05) (width 0.2) (layer "B.Cu") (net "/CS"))
 (segment (start 92.9 86.05) (end 92.9 59.131) (width 0.2) (layer "B.Cu") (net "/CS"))
 (segment (start 92.9 59.131) (end 94.275 57.756) (width 0.2) (layer "B.Cu") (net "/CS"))
 (segment (start 95.11 57.756) (end 94.275 57.756) (width 0.2) (layer "B.Cu") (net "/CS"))
 (segment (start 95.11 55.216) (end 94.03237 55.216) (width 0.2) (layer "B.Cu") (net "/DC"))
 (segment (start 92.5 88.19) (end 107.31 103) (width 0.2) (layer "B.Cu") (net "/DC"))
 (segment (start 94.03237 55.216) (end 92.5 56.74837) (width 0.2) (layer "B.Cu") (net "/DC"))
 (segment (start 92.5 56.74837) (end 92.5 88.19) (width 0.2) (layer "B.Cu") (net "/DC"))
 (segment (start 92 92.77) (end 102.23 103) (width 0.2) (layer "B.Cu") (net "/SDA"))
 (segment (start 95.11 52.676) (end 94.03237 52.676) (width 0.2) (layer "B.Cu") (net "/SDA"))
 (segment (start 92 54.70837) (end 92 92.77) (width 0.2) (layer "B.Cu") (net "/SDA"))
 (segment (start 94.03237 52.676) (end 92 54.70837) (width 0.2) (layer "B.Cu") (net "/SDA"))
 (segment (start 95.11 50.136) (end 94.03237 50.136) (width 0.2) (layer "B.Cu") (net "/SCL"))
 (segment (start 94.03237 50.136) (end 91.5 52.66837) (width 0.2) (layer "B.Cu") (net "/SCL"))
 (segment (start 91.5 52.66837) (end 91.5 94.81) (width 0.2) (layer "B.Cu") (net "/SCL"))
 (segment (start 91.5 94.81) (end 99.69 103) (width 0.2) (layer "B.Cu") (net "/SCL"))
 (segment (start 103.27 104.5) (end 104.77 103) (width 0.2) (layer "F.Cu") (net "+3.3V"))
 (segment (start 95.65 101.5) (end 97.15 103) (width 0.2) (layer "F.Cu") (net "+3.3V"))
 (segment (start 78 64.706) (end 78 89.5) (width 0.2) (layer "F.Cu") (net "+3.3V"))
 (segment (start 78 89.5) (end 90 101.5) (width 0.2) (layer "F.Cu") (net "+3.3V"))
 (segment (start 90 101.5) (end 95.65 101.5) (width 0.2) (layer "F.Cu") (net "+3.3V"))
 (segment (start 98.65 104.5) (end 103.27 104.5) (width 0.2) (layer "F.Cu") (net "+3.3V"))
 (segment (start 97.15 103) (end 98.65 104.5) (width 0.2) (layer "F.Cu") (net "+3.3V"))
 (segment (start 95.11 47.596) (end 78 64.706) (width 0.2) (layer "F.Cu") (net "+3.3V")))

